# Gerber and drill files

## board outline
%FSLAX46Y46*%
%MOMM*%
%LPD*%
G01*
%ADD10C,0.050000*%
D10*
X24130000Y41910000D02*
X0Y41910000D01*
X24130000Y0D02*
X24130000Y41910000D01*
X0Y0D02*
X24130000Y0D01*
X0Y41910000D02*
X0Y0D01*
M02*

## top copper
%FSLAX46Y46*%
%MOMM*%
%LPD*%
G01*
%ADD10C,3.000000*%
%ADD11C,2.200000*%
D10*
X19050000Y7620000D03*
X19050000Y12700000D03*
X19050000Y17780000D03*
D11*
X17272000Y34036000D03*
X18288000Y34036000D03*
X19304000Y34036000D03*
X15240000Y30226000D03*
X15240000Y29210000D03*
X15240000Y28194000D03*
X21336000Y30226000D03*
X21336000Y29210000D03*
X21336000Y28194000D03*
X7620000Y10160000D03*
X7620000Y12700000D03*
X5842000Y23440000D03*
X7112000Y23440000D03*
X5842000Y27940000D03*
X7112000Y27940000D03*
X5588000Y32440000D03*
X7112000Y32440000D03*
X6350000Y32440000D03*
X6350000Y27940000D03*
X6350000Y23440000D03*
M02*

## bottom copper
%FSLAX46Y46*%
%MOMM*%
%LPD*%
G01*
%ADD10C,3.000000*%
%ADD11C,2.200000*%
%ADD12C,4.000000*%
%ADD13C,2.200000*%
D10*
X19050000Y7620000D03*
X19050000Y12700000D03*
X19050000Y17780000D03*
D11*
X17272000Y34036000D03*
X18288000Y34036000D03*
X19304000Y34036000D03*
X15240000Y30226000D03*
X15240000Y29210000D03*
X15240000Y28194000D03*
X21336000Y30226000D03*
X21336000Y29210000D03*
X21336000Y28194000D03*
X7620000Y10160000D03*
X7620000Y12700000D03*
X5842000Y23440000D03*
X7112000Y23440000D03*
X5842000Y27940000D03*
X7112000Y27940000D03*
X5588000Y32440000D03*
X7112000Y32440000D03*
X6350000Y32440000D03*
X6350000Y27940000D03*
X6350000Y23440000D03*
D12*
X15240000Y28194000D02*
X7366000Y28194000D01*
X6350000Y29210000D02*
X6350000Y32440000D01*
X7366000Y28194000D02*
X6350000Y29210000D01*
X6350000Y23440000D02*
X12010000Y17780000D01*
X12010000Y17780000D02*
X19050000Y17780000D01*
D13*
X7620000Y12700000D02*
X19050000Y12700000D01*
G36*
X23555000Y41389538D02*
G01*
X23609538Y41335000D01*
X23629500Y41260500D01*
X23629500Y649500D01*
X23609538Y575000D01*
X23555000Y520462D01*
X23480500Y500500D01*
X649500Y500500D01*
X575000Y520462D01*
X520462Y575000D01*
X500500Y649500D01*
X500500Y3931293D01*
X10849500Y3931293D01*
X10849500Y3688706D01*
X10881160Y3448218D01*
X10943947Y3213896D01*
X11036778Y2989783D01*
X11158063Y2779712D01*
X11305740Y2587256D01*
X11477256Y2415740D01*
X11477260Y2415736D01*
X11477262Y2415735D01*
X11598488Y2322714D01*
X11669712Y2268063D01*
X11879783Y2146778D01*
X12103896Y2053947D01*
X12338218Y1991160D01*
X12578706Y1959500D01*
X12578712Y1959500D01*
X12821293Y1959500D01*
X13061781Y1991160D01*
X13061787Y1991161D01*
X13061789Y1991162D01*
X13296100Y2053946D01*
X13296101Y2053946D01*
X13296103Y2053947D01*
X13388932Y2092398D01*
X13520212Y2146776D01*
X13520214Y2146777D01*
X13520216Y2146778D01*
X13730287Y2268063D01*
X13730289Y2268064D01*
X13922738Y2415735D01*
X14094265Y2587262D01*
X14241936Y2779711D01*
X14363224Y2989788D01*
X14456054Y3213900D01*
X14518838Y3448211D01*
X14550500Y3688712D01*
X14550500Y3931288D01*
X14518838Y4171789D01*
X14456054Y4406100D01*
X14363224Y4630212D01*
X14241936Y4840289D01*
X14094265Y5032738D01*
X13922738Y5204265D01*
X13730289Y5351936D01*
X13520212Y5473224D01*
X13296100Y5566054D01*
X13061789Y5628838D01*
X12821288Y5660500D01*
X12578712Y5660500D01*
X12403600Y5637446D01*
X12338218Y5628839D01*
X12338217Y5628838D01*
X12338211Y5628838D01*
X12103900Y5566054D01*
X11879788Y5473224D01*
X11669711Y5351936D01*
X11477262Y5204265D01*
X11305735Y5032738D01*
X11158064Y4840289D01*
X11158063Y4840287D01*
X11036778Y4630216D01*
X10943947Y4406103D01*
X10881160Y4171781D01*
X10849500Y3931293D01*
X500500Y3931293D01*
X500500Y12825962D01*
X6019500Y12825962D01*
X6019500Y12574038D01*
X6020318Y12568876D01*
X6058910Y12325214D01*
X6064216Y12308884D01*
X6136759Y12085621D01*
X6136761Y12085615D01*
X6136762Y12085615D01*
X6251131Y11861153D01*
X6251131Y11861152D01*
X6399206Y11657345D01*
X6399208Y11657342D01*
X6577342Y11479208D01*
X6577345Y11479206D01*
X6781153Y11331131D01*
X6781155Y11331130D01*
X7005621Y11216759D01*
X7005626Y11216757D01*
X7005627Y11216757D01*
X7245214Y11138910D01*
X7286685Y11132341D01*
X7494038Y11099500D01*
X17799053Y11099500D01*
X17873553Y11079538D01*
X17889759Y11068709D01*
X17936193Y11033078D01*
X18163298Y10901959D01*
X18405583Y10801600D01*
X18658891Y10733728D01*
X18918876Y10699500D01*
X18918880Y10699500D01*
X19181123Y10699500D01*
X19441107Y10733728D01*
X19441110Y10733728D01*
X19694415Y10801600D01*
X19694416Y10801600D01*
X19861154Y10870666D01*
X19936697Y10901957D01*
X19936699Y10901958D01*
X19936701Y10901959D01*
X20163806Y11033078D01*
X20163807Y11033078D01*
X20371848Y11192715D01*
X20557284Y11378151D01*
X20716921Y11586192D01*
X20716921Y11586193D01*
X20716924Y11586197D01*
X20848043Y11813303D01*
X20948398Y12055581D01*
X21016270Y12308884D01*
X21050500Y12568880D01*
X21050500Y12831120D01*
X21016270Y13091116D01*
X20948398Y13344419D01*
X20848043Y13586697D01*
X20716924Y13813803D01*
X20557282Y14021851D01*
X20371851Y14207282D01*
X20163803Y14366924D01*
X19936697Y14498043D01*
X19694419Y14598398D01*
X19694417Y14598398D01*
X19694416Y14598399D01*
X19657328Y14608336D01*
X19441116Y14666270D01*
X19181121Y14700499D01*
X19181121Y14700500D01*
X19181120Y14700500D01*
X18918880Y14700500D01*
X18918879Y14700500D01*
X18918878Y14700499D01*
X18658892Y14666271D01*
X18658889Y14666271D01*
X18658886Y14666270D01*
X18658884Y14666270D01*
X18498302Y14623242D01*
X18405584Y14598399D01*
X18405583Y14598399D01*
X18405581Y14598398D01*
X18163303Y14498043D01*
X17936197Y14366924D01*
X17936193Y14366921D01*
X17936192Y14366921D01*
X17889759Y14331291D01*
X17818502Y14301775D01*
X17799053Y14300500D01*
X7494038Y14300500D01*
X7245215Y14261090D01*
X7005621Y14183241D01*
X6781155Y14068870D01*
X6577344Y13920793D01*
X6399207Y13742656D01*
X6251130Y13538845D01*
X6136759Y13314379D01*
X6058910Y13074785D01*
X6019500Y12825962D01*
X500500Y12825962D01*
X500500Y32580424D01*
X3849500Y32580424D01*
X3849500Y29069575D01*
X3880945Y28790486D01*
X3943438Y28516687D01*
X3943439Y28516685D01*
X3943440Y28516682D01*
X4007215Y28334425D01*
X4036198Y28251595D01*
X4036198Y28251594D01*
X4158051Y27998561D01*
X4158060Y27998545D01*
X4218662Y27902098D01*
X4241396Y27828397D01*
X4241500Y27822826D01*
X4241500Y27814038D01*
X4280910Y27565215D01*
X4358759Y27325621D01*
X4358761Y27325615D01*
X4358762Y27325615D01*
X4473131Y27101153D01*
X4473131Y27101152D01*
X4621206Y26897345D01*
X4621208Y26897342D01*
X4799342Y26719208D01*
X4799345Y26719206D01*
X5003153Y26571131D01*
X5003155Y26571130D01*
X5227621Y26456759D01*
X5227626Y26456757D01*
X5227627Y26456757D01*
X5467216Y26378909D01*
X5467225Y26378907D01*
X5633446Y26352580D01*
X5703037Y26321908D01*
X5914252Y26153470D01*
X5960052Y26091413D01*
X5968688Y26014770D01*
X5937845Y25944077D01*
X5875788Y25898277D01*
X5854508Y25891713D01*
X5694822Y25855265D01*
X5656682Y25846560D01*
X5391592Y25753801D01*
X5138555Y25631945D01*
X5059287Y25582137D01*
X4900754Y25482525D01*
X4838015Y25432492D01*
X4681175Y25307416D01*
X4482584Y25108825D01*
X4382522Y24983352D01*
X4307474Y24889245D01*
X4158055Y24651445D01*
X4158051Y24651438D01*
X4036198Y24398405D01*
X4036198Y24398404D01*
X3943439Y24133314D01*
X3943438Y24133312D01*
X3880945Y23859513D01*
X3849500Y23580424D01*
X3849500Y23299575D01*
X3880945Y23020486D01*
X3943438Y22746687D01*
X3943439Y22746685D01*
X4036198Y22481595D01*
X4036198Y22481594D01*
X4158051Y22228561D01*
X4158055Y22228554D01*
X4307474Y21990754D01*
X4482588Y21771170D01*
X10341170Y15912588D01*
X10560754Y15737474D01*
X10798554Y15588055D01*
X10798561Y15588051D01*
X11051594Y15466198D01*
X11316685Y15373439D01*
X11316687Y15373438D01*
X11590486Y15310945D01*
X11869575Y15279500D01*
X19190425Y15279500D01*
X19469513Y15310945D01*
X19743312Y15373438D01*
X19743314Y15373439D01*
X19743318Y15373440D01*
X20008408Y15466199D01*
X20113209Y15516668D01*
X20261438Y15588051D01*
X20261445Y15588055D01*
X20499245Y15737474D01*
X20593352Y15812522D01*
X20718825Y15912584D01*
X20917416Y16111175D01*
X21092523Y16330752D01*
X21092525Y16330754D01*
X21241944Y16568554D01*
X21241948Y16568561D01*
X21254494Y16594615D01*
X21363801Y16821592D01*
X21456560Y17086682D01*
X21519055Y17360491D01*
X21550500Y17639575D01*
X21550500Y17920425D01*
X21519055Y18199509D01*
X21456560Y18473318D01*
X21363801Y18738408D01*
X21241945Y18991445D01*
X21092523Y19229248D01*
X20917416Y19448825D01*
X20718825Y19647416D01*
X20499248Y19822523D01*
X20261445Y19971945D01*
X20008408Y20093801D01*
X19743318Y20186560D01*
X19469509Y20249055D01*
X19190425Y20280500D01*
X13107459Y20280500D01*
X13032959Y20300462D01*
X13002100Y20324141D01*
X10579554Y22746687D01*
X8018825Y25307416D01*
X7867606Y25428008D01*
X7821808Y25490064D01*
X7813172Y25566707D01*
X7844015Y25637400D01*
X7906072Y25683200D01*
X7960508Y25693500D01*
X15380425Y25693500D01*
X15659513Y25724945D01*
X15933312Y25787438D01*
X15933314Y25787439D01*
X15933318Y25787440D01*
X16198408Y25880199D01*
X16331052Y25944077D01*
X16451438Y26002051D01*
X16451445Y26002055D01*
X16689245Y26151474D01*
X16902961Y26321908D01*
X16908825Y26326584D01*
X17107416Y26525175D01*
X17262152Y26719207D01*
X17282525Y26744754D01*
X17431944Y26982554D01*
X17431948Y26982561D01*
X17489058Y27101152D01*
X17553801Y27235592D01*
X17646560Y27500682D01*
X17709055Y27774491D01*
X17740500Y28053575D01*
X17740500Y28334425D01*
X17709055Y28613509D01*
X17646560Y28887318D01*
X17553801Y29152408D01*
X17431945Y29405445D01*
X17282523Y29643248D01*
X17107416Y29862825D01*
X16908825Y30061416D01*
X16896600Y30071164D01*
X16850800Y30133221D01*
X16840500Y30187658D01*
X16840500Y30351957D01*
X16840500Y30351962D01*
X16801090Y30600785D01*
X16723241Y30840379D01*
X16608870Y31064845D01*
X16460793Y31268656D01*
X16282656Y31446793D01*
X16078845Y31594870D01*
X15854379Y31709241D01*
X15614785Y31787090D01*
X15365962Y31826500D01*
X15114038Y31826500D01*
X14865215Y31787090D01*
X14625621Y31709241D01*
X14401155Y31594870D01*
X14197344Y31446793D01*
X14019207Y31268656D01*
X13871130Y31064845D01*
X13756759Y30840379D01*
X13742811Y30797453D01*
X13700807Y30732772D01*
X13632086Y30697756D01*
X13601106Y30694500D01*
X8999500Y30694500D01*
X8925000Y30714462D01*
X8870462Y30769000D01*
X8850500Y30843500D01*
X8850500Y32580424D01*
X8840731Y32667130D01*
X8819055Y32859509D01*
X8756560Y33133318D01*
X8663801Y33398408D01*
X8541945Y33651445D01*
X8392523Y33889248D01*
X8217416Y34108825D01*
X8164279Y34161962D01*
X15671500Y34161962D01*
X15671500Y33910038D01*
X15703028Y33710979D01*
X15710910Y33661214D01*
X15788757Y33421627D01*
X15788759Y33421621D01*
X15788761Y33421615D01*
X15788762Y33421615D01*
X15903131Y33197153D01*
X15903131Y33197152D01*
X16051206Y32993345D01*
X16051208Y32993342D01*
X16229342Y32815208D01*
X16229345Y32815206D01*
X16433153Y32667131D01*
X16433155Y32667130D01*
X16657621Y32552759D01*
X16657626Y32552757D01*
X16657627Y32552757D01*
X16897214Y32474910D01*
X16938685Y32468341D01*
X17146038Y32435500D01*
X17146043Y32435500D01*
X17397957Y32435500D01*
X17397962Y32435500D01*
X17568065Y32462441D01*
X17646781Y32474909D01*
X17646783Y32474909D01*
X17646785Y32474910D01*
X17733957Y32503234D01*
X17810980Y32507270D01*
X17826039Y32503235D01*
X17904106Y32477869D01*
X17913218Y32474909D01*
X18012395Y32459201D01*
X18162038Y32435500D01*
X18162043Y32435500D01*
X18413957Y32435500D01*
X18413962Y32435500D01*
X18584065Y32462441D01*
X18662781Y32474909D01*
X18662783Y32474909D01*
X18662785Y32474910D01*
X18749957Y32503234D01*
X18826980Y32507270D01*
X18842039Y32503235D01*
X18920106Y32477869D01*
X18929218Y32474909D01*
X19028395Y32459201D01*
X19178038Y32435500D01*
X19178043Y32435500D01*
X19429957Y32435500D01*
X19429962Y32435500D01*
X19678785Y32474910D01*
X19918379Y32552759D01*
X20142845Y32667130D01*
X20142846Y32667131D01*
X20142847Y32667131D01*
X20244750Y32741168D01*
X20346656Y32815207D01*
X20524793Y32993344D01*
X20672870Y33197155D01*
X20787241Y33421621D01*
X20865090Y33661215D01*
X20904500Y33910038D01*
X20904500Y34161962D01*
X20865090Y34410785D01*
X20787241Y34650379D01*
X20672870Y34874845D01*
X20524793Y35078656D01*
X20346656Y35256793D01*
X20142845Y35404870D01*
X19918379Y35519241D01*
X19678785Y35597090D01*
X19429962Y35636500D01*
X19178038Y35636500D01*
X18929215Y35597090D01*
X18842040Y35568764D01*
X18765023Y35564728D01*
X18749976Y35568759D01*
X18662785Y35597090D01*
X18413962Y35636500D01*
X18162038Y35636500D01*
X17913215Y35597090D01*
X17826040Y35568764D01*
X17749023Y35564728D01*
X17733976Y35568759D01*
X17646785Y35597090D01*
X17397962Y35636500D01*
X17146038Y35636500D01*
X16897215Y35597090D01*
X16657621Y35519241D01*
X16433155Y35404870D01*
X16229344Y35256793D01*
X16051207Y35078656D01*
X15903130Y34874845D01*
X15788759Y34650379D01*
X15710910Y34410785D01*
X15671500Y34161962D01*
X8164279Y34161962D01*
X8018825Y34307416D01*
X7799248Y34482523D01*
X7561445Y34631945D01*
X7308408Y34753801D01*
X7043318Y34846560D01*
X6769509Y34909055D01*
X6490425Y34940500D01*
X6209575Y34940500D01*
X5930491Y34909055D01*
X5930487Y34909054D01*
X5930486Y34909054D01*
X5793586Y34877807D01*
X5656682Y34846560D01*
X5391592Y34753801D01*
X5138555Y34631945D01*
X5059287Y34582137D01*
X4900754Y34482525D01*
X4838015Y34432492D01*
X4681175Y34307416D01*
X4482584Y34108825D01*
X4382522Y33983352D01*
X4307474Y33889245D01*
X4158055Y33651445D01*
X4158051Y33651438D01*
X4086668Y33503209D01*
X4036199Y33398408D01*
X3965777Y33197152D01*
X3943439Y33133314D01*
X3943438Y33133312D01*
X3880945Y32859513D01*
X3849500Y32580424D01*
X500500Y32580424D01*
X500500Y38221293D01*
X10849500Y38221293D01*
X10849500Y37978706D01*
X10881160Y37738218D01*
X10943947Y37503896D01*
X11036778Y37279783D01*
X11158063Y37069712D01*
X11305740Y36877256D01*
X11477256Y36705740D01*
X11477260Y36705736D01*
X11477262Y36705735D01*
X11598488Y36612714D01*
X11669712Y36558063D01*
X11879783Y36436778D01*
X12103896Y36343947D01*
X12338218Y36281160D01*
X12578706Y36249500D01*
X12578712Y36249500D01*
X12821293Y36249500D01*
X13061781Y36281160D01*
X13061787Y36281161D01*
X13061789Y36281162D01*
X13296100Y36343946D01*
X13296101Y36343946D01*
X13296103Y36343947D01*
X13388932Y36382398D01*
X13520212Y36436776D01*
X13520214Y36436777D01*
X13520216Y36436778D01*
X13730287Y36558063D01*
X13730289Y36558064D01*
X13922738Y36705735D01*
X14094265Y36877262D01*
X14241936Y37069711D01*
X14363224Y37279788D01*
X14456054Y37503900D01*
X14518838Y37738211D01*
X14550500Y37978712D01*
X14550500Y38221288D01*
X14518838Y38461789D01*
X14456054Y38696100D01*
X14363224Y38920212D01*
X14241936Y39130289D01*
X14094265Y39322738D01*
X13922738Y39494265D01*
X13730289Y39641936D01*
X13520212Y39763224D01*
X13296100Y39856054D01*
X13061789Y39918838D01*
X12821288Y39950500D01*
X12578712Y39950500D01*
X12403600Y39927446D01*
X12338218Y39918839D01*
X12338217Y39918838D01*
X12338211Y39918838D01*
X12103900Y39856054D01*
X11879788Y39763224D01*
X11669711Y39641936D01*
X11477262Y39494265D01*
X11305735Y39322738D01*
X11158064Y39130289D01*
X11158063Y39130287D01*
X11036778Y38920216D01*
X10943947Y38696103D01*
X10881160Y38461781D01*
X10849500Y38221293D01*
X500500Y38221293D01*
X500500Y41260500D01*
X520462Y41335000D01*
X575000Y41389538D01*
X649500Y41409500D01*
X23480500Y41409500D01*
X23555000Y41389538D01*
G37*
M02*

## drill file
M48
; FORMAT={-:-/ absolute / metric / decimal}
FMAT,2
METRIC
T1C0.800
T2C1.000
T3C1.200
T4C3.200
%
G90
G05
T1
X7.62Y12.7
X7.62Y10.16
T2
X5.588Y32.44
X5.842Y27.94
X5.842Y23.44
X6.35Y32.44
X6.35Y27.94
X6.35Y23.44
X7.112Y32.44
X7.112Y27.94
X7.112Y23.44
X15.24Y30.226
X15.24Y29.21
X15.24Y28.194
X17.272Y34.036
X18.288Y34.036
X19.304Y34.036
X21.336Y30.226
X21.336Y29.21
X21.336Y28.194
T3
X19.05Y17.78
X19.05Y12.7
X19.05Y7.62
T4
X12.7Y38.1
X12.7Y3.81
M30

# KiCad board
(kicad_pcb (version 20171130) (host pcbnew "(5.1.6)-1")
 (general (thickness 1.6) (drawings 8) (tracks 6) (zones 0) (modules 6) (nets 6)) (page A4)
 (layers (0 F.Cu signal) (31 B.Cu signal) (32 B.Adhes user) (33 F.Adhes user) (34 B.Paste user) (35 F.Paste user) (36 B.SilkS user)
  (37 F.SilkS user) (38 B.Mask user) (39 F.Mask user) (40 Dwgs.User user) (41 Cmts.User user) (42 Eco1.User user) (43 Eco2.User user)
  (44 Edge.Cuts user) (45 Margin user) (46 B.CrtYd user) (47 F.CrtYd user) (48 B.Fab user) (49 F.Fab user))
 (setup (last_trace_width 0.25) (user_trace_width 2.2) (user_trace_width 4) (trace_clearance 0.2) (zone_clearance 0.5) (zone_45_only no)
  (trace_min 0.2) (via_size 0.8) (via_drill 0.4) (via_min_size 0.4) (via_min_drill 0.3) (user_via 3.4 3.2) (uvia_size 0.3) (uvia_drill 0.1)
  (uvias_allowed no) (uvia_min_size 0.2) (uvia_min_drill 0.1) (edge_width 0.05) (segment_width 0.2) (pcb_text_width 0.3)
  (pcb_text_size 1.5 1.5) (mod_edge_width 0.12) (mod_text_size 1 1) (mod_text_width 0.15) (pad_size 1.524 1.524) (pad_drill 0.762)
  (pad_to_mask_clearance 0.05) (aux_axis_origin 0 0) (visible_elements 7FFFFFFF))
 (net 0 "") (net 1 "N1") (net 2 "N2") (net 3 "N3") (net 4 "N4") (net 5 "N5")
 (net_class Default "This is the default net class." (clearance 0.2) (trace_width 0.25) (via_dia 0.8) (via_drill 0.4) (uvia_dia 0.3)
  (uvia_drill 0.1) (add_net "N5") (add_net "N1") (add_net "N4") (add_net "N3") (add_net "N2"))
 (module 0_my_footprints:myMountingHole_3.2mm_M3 (layer F.Cu) (at 12.7 -3.81)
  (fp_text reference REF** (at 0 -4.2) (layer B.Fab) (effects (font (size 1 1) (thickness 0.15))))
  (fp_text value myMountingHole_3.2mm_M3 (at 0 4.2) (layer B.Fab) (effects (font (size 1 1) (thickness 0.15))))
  (pad "" np_thru_hole circle (at 0 0) (size 3.2 3.2) (drill 3.2) (layers *.Cu *.Mask)))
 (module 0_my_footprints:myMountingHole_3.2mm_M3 (layer F.Cu) (at 12.7 -38.1)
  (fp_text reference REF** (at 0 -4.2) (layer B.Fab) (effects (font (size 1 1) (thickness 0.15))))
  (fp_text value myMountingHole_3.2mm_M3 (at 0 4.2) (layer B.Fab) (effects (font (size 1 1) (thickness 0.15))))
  (pad "" np_thru_hole circle (at 0 0) (size 3.2 3.2) (drill 3.2) (layers *.Cu *.Mask)))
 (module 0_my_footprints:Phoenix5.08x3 (layer F.Cu) (at 19.05 -12.7 270)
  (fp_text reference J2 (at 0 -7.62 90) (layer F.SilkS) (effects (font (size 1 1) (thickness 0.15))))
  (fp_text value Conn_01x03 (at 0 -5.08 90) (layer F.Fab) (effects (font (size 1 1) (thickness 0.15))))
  (pad 3 thru_hole circle (at 5.08 0 270) (size 3 3) (drill 1.2) (layers *.Cu *.Mask) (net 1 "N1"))
  (pad 2 thru_hole circle (at 0 0 270) (size 3 3) (drill 1.2) (layers *.Cu *.Mask) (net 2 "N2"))
  (pad 1 thru_hole circle (at -5.08 0 270) (size 3 3) (drill 1.2) (layers *.Cu *.Mask) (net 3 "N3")))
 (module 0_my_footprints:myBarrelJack (layer F.Cu) (at 15.24 -29.21 180)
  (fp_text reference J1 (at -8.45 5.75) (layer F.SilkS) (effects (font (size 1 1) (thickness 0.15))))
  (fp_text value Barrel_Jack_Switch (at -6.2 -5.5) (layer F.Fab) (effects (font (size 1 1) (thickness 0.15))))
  (pad 3 thru_hole circle (at -2.032 4.826 180) (size 2.2 2.2) (drill 1) (layers *.Cu *.Mask) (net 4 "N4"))
  (pad 3 thru_hole circle (at -3.048 4.826 180) (size 2.2 2.2) (drill 1) (layers *.Cu *.Mask) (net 4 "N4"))
  (pad 3 thru_hole circle (at -4.064 4.826 180) (size 2.2 2.2) (drill 1) (layers *.Cu *.Mask) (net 4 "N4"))
  (pad 1 thru_hole circle (at 0 1.016 180) (size 2.2 2.2) (drill 1) (layers *.Cu *.Mask) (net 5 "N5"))
  (pad 1 thru_hole circle (at 0 0 180) (size 2.2 2.2) (drill 1) (layers *.Cu *.Mask) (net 5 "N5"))
  (pad 1 thru_hole circle (at 0 -1.016 180) (size 2.2 2.2) (drill 1) (layers *.Cu *.Mask) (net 5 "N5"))
  (pad 2 thru_hole circle (at -6.096 1.016 180) (size 2.2 2.2) (drill 1) (layers *.Cu *.Mask) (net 1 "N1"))
  (pad 2 thru_hole circle (at -6.096 0 180) (size 2.2 2.2) (drill 1) (layers *.Cu *.Mask) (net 1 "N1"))
  (pad 2 thru_hole circle (at -6.096 -1.016 180) (size 2.2 2.2) (drill 1) (layers *.Cu *.Mask) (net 1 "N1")))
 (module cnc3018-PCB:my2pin (layer F.Cu) (at 7.62 -10.16 90)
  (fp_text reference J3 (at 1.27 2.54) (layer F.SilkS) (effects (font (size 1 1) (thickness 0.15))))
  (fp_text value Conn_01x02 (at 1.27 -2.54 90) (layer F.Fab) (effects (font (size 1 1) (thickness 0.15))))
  (pad 1 thru_hole circle (at 0 0 90) (size 2.2 2.2) (drill 0.8) (layers *.Cu *.Mask) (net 1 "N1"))
  (pad 2 thru_hole circle (at 2.54 0 90) (size 2.2 2.2) (drill 0.8) (layers *.Cu *.Mask) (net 2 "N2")))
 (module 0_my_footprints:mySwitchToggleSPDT (layer F.Cu) (at 6.35 -27.94 270)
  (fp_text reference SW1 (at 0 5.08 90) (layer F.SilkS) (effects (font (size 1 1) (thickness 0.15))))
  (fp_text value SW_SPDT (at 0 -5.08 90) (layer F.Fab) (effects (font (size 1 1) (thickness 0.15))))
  (pad 3 thru_hole circle (at 4.5 0.508 270) (size 2.2 2.2) (drill 1) (layers *.Cu *.Mask) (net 3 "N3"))
  (pad 3 thru_hole circle (at 4.5 -0.762 270) (size 2.2 2.2) (drill 1) (layers *.Cu *.Mask) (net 3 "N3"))
  (pad 2 thru_hole circle (at 0 0.508 270) (size 2.2 2.2) (drill 1) (layers *.Cu *.Mask) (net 5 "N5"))
  (pad 2 thru_hole circle (at 0 -0.762 270) (size 2.2 2.2) (drill 1) (layers *.Cu *.Mask) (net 5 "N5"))
  (pad 1 thru_hole circle (at -4.5 0.762 270) (size 2.2 2.2) (drill 1) (layers *.Cu *.Mask) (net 5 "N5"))
  (pad 1 thru_hole circle (at -4.5 -0.762 270) (size 2.2 2.2) (drill 1) (layers *.Cu *.Mask) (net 5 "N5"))
  (pad 1 thru_hole circle (at -4.5 0 270) (size 2.2 2.2) (drill 1) (layers *.Cu *.Mask) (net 5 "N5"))
  (pad 2 thru_hole circle (at 0 0 270) (size 2.2 2.2) (drill 1) (layers *.Cu *.Mask) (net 5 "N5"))
  (pad 3 thru_hole circle (at 4.5 0 270) (size 2.2 2.2) (drill 1) (layers *.Cu *.Mask) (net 3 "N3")))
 (gr_line (start 24.13 -41.91) (end 0 -41.91) (layer Edge.Cuts) (width 0.05))
 (gr_line (start 24.13 0) (end 24.13 -41.91) (layer Edge.Cuts) (width 0.05))
 (gr_line (start 0 0) (end 24.13 0) (layer Edge.Cuts) (width 0.05))
 (gr_line (start 0 -41.91) (end 0 0) (layer Edge.Cuts) (width 0.05))
 (segment (start 15.24 -28.194) (end 7.366 -28.194) (width 4) (layer B.Cu) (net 5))
 (segment (start 6.35 -29.21) (end 6.35 -32.44) (width 4) (layer B.Cu) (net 5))
 (segment (start 7.366 -28.194) (end 6.35 -29.21) (width 4) (layer B.Cu) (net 5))
 (segment (start 6.35 -23.44) (end 12.01 -17.78) (width 4) (layer B.Cu) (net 3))
 (segment (start 12.01 -17.78) (end 19.05 -17.78) (width 4) (layer B.Cu) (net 3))
 (segment (start 7.62 -12.7) (end 19.05 -12.7) (width 2.2) (layer B.Cu) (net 2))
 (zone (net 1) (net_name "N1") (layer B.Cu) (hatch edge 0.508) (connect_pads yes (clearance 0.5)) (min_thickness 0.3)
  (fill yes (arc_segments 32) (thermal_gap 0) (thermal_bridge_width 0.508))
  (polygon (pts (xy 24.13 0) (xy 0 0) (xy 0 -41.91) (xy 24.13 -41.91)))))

